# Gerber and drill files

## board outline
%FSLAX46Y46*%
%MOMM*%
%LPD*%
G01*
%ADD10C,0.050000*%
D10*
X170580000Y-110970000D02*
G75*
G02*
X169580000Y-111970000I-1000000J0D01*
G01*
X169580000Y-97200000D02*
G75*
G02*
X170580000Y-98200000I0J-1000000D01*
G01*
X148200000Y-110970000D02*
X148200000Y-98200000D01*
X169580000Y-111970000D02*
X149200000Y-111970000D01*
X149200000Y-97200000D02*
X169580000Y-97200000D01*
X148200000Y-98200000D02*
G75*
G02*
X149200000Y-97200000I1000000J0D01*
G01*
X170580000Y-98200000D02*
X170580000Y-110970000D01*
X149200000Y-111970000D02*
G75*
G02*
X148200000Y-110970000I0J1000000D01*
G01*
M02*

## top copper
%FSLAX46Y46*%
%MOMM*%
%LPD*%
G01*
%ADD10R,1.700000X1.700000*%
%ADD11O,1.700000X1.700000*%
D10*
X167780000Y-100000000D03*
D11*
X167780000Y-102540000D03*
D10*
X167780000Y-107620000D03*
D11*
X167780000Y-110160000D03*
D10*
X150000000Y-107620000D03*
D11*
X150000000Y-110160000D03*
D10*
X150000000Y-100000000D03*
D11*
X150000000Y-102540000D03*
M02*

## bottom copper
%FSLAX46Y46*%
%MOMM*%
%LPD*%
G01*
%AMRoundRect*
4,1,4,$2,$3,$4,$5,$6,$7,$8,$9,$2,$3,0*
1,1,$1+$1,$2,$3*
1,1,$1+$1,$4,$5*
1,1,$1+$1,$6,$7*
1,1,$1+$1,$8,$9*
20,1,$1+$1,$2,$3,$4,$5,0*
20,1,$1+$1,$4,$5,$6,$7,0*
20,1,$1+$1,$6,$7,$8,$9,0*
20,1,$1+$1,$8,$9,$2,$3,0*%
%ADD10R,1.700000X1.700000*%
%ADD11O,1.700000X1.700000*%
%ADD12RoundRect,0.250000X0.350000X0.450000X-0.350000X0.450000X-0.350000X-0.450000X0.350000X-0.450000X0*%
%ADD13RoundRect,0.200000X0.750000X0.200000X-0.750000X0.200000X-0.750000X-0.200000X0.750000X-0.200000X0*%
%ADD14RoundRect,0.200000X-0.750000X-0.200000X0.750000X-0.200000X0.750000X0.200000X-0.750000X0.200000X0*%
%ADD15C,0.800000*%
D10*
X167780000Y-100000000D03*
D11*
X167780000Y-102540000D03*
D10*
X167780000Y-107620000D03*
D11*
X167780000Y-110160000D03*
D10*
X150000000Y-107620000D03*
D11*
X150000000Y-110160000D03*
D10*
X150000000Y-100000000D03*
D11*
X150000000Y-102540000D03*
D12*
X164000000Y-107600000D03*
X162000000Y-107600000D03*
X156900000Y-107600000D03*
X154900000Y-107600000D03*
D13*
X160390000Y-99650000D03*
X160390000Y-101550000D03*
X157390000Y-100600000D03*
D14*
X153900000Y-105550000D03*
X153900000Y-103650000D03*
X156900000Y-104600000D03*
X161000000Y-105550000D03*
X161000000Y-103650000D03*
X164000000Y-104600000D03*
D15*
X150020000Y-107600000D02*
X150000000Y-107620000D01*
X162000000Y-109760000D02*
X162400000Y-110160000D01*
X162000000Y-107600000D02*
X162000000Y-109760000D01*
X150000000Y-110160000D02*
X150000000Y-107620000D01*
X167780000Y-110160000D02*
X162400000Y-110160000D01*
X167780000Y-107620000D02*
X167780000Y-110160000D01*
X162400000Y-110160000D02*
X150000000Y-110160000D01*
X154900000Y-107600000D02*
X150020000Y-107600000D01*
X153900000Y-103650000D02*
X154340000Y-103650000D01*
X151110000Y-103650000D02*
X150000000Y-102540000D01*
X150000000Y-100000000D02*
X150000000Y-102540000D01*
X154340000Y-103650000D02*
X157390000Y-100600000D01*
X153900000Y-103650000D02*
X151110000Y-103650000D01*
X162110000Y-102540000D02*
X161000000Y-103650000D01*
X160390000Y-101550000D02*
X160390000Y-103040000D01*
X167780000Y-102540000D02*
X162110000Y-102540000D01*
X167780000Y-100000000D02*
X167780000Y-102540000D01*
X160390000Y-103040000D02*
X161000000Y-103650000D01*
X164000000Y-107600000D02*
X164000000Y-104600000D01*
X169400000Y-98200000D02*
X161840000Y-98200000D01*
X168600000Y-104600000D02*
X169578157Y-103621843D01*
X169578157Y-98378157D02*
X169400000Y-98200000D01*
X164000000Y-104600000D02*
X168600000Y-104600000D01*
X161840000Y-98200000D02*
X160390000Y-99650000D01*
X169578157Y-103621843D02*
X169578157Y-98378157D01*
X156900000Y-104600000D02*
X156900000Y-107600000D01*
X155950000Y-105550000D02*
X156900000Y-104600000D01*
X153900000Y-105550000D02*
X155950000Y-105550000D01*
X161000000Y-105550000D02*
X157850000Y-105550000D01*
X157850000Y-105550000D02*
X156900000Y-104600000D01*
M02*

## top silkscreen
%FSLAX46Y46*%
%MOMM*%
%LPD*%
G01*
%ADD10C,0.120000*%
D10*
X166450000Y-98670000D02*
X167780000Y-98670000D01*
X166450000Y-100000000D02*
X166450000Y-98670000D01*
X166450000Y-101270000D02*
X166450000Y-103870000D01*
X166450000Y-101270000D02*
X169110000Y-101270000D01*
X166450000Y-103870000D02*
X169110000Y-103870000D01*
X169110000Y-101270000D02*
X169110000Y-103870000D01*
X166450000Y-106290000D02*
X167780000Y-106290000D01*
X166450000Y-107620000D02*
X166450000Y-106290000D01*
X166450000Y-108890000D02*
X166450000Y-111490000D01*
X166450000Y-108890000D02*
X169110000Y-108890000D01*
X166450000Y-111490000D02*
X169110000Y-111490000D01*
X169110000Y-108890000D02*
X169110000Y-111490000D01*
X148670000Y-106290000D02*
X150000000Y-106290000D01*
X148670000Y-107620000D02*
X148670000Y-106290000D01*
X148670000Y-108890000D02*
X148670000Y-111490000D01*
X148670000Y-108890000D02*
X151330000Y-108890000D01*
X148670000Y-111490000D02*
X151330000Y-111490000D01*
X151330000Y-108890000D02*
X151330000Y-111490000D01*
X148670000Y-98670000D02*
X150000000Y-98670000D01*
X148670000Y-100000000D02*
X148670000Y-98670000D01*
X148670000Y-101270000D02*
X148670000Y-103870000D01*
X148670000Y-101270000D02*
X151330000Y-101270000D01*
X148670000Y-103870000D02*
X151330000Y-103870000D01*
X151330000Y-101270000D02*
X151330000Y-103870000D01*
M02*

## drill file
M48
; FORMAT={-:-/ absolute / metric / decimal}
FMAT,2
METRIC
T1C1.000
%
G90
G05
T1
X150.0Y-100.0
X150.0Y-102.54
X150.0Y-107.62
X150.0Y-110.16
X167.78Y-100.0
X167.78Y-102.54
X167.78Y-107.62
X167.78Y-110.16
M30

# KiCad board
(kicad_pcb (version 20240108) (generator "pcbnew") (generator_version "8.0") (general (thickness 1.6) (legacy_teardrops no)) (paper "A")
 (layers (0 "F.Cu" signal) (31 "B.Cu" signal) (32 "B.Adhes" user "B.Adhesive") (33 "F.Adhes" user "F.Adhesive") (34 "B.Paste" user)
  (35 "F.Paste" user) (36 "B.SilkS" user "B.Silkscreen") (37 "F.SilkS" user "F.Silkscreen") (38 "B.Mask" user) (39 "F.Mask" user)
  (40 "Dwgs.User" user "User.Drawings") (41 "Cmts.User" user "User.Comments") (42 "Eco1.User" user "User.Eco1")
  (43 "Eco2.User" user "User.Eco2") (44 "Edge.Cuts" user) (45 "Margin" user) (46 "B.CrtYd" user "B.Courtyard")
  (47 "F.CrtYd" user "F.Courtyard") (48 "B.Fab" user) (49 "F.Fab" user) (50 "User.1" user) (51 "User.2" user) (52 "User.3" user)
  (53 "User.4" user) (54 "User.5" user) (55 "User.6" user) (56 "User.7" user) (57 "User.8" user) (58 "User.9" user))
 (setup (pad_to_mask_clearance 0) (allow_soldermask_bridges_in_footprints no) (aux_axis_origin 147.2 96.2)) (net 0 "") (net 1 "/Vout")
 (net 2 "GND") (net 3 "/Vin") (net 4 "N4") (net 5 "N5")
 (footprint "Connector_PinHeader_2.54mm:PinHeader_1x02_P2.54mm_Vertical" (layer "F.Cu") (at 167.78 100)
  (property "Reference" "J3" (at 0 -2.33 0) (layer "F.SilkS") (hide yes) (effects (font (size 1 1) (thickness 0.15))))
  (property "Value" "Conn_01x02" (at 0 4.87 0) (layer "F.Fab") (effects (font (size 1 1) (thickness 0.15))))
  (fp_line (start -1.33 -1.33) (end 0 -1.33) (stroke (width 0.12) (type solid)) (layer "F.SilkS"))
  (fp_line (start -1.33 0) (end -1.33 -1.33) (stroke (width 0.12) (type solid)) (layer "F.SilkS"))
  (fp_line (start -1.33 1.27) (end -1.33 3.87) (stroke (width 0.12) (type solid)) (layer "F.SilkS"))
  (fp_line (start -1.33 1.27) (end 1.33 1.27) (stroke (width 0.12) (type solid)) (layer "F.SilkS"))
  (fp_line (start -1.33 3.87) (end 1.33 3.87) (stroke (width 0.12) (type solid)) (layer "F.SilkS"))
  (fp_line (start 1.33 1.27) (end 1.33 3.87) (stroke (width 0.12) (type solid)) (layer "F.SilkS"))
  (pad "1" thru_hole rect (at 0 0) (size 1.7 1.7) (drill 1) (layers "*.Cu" "*.Mask") (remove_unused_layers no) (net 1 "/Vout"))
  (pad "2" thru_hole oval (at 0 2.54) (size 1.7 1.7) (drill 1) (layers "*.Cu" "*.Mask") (remove_unused_layers no) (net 1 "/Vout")))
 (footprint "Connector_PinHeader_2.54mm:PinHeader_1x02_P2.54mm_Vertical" (layer "F.Cu") (at 167.78 107.62)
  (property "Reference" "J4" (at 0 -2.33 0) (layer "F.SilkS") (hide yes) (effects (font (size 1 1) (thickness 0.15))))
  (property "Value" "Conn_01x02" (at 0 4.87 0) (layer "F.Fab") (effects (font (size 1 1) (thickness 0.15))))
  (fp_line (start -1.33 -1.33) (end 0 -1.33) (stroke (width 0.12) (type solid)) (layer "F.SilkS"))
  (fp_line (start -1.33 0) (end -1.33 -1.33) (stroke (width 0.12) (type solid)) (layer "F.SilkS"))
  (fp_line (start -1.33 1.27) (end -1.33 3.87) (stroke (width 0.12) (type solid)) (layer "F.SilkS"))
  (fp_line (start -1.33 1.27) (end 1.33 1.27) (stroke (width 0.12) (type solid)) (layer "F.SilkS"))
  (fp_line (start -1.33 3.87) (end 1.33 3.87) (stroke (width 0.12) (type solid)) (layer "F.SilkS"))
  (fp_line (start 1.33 1.27) (end 1.33 3.87) (stroke (width 0.12) (type solid)) (layer "F.SilkS"))
  (pad "1" thru_hole rect (at 0 0) (size 1.7 1.7) (drill 1) (layers "*.Cu" "*.Mask") (remove_unused_layers no) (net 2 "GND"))
  (pad "2" thru_hole oval (at 0 2.54) (size 1.7 1.7) (drill 1) (layers "*.Cu" "*.Mask") (remove_unused_layers no) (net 2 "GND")))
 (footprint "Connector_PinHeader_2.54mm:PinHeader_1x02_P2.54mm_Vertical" (layer "F.Cu") (at 150 107.62)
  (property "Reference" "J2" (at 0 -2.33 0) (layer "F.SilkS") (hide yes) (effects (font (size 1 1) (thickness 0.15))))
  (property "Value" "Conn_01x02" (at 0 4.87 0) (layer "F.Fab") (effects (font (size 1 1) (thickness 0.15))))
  (fp_line (start -1.33 -1.33) (end 0 -1.33) (stroke (width 0.12) (type solid)) (layer "F.SilkS"))
  (fp_line (start -1.33 0) (end -1.33 -1.33) (stroke (width 0.12) (type solid)) (layer "F.SilkS"))
  (fp_line (start -1.33 1.27) (end -1.33 3.87) (stroke (width 0.12) (type solid)) (layer "F.SilkS"))
  (fp_line (start -1.33 1.27) (end 1.33 1.27) (stroke (width 0.12) (type solid)) (layer "F.SilkS"))
  (fp_line (start -1.33 3.87) (end 1.33 3.87) (stroke (width 0.12) (type solid)) (layer "F.SilkS"))
  (fp_line (start 1.33 1.27) (end 1.33 3.87) (stroke (width 0.12) (type solid)) (layer "F.SilkS"))
  (pad "1" thru_hole rect (at 0 0) (size 1.7 1.7) (drill 1) (layers "*.Cu" "*.Mask") (remove_unused_layers no) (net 2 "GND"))
  (pad "2" thru_hole oval (at 0 2.54) (size 1.7 1.7) (drill 1) (layers "*.Cu" "*.Mask") (remove_unused_layers no) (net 2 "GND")))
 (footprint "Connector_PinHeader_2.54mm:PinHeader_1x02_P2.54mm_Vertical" (layer "F.Cu") (at 150 100)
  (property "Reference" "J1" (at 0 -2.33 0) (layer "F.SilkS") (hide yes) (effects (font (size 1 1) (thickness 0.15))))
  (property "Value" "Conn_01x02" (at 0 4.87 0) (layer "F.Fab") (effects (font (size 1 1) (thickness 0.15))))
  (fp_line (start -1.33 -1.33) (end 0 -1.33) (stroke (width 0.12) (type solid)) (layer "F.SilkS"))
  (fp_line (start -1.33 0) (end -1.33 -1.33) (stroke (width 0.12) (type solid)) (layer "F.SilkS"))
  (fp_line (start -1.33 1.27) (end -1.33 3.87) (stroke (width 0.12) (type solid)) (layer "F.SilkS"))
  (fp_line (start -1.33 1.27) (end 1.33 1.27) (stroke (width 0.12) (type solid)) (layer "F.SilkS"))
  (fp_line (start -1.33 3.87) (end 1.33 3.87) (stroke (width 0.12) (type solid)) (layer "F.SilkS"))
  (fp_line (start 1.33 1.27) (end 1.33 3.87) (stroke (width 0.12) (type solid)) (layer "F.SilkS"))
  (pad "1" thru_hole rect (at 0 0) (size 1.7 1.7) (drill 1) (layers "*.Cu" "*.Mask") (remove_unused_layers no) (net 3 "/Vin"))
  (pad "2" thru_hole oval (at 0 2.54) (size 1.7 1.7) (drill 1) (layers "*.Cu" "*.Mask") (remove_unused_layers no) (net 3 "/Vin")))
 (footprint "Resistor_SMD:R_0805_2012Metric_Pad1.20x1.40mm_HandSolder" (layer "B.Cu") (at 163 107.6 180)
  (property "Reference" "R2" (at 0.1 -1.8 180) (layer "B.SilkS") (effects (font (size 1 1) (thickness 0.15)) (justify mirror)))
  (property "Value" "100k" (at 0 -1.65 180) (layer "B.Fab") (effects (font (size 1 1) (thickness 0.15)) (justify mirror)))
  (pad "1" smd roundrect (at -1 0 180) (size 1.2 1.4) (layers "B.Cu" "B.Paste" "B.Mask") (roundrect_rratio 0.208333) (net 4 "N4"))
  (pad "2" smd roundrect (at 1 0 180) (size 1.2 1.4) (layers "B.Cu" "B.Paste" "B.Mask") (roundrect_rratio 0.208333) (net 2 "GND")))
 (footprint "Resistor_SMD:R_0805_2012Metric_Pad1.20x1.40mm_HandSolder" (layer "B.Cu") (at 155.9 107.6 180)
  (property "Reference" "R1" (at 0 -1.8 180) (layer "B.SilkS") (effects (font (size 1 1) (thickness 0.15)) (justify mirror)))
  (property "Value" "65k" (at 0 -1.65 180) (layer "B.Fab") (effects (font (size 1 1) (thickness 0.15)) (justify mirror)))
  (pad "1" smd roundrect (at -1 0 180) (size 1.2 1.4) (layers "B.Cu" "B.Paste" "B.Mask") (roundrect_rratio 0.208333) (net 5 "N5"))
  (pad "2" smd roundrect (at 1 0 180) (size 1.2 1.4) (layers "B.Cu" "B.Paste" "B.Mask") (roundrect_rratio 0.208333) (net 2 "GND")))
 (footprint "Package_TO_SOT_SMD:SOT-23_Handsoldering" (layer "B.Cu") (at 158.89 100.6 180)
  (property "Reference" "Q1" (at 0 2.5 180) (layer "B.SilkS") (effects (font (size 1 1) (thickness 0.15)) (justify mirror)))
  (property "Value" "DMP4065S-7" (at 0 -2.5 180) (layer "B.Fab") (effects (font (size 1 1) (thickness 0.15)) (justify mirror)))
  (pad "1" smd roundrect (at -1.5 0.95 180) (size 1.9 0.8) (layers "B.Cu" "B.Paste" "B.Mask") (roundrect_rratio 0.25) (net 4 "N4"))
  (pad "2" smd roundrect (at -1.5 -0.95 180) (size 1.9 0.8) (layers "B.Cu" "B.Paste" "B.Mask") (roundrect_rratio 0.25) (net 1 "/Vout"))
  (pad "3" smd roundrect (at 1.5 0 180) (size 1.9 0.8) (layers "B.Cu" "B.Paste" "B.Mask") (roundrect_rratio 0.25) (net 3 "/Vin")))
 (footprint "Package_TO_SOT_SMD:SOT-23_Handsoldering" (layer "B.Cu") (at 155.4 104.6)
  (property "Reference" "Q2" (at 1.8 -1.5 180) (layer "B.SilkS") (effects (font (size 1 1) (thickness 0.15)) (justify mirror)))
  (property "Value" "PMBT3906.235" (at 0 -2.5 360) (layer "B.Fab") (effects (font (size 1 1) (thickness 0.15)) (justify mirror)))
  (pad "1" smd roundrect (at -1.5 0.95) (size 1.9 0.8) (layers "B.Cu" "B.Paste" "B.Mask") (roundrect_rratio 0.25) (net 5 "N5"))
  (pad "2" smd roundrect (at -1.5 -0.95) (size 1.9 0.8) (layers "B.Cu" "B.Paste" "B.Mask") (roundrect_rratio 0.25) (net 3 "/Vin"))
  (pad "3" smd roundrect (at 1.5 0) (size 1.9 0.8) (layers "B.Cu" "B.Paste" "B.Mask") (roundrect_rratio 0.25) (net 5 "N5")))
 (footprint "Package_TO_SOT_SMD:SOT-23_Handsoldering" (layer "B.Cu") (at 162.5 104.6)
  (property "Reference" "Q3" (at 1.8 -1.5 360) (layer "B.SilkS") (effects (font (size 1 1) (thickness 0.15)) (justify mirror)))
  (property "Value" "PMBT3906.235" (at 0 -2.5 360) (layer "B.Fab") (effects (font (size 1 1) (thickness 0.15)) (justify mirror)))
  (pad "1" smd roundrect (at -1.5 0.95) (size 1.9 0.8) (layers "B.Cu" "B.Paste" "B.Mask") (roundrect_rratio 0.25) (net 5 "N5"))
  (pad "2" smd roundrect (at -1.5 -0.95) (size 1.9 0.8) (layers "B.Cu" "B.Paste" "B.Mask") (roundrect_rratio 0.25) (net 1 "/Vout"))
  (pad "3" smd roundrect (at 1.5 0) (size 1.9 0.8) (layers "B.Cu" "B.Paste" "B.Mask") (roundrect_rratio 0.25) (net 4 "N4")))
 (gr_arc (start 170.58 110.97) (mid 170.287107 111.677107) (end 169.58 111.97) (stroke (width 0.05) (type default)) (layer "Edge.Cuts"))
 (gr_arc (start 169.58 97.2) (mid 170.287107 97.492893) (end 170.58 98.2) (stroke (width 0.05) (type default)) (layer "Edge.Cuts"))
 (gr_line (start 148.2 110.97) (end 148.2 98.2) (stroke (width 0.05) (type default)) (layer "Edge.Cuts"))
 (gr_line (start 169.58 111.97) (end 149.2 111.97) (stroke (width 0.05) (type default)) (layer "Edge.Cuts"))
 (gr_line (start 149.2 97.2) (end 169.58 97.2) (stroke (width 0.05) (type default)) (layer "Edge.Cuts"))
 (gr_arc (start 148.2 98.2) (mid 148.492893 97.492893) (end 149.2 97.2) (stroke (width 0.05) (type default)) (layer "Edge.Cuts"))
 (gr_line (start 170.58 98.2) (end 170.58 110.97) (stroke (width 0.05) (type default)) (layer "Edge.Cuts"))
 (gr_arc (start 149.2 111.97) (mid 148.492893 111.677107) (end 148.2 110.97) (stroke (width 0.05) (type default)) (layer "Edge.Cuts"))
 (segment (start 150.02 107.6) (end 150 107.62) (width 0.8) (layer "B.Cu") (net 2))
 (segment (start 162 109.76) (end 162.4 110.16) (width 0.8) (layer "B.Cu") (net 2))
 (segment (start 162 107.6) (end 162 109.76) (width 0.8) (layer "B.Cu") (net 2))
 (segment (start 150 110.16) (end 150 107.62) (width 0.8) (layer "B.Cu") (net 2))
 (segment (start 167.78 110.16) (end 162.4 110.16) (width 0.8) (layer "B.Cu") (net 2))
 (segment (start 167.78 107.62) (end 167.78 110.16) (width 0.8) (layer "B.Cu") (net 2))
 (segment (start 162.4 110.16) (end 150 110.16) (width 0.8) (layer "B.Cu") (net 2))
 (segment (start 154.9 107.6) (end 150.02 107.6) (width 0.8) (layer "B.Cu") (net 2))
 (segment (start 153.9 103.65) (end 154.34 103.65) (width 0.8) (layer "B.Cu") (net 3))
 (segment (start 151.11 103.65) (end 150 102.54) (width 0.8) (layer "B.Cu") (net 3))
 (segment (start 150 100) (end 150 102.54) (width 0.8) (layer "B.Cu") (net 3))
 (segment (start 154.34 103.65) (end 157.39 100.6) (width 0.8) (layer "B.Cu") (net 3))
 (segment (start 153.9 103.65) (end 151.11 103.65) (width 0.8) (layer "B.Cu") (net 3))
 (segment (start 162.11 102.54) (end 161 103.65) (width 0.8) (layer "B.Cu") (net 1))
 (segment (start 160.39 101.55) (end 160.39 103.04) (width 0.8) (layer "B.Cu") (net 1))
 (segment (start 167.78 102.54) (end 162.11 102.54) (width 0.8) (layer "B.Cu") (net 1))
 (segment (start 167.78 100) (end 167.78 102.54) (width 0.8) (layer "B.Cu") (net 1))
 (segment (start 160.39 103.04) (end 161 103.65) (width 0.8) (layer "B.Cu") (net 1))
 (segment (start 164 107.6) (end 164 104.6) (width 0.8) (layer "B.Cu") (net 4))
 (segment (start 169.4 98.2) (end 161.84 98.2) (width 0.8) (layer "B.Cu") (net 4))
 (segment (start 168.6 104.6) (end 169.578157 103.621843) (width 0.8) (layer "B.Cu") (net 4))
 (segment (start 169.578157 98.378157) (end 169.4 98.2) (width 0.8) (layer "B.Cu") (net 4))
 (segment (start 164 104.6) (end 168.6 104.6) (width 0.8) (layer "B.Cu") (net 4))
 (segment (start 161.84 98.2) (end 160.39 99.65) (width 0.8) (layer "B.Cu") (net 4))
 (segment (start 169.578157 103.621843) (end 169.578157 98.378157) (width 0.8) (layer "B.Cu") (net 4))
 (segment (start 156.9 104.6) (end 156.9 107.6) (width 0.8) (layer "B.Cu") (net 5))
 (segment (start 155.95 105.55) (end 156.9 104.6) (width 0.8) (layer "B.Cu") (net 5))
 (segment (start 153.9 105.55) (end 155.95 105.55) (width 0.8) (layer "B.Cu") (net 5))
 (segment (start 161 105.55) (end 157.85 105.55) (width 0.8) (layer "B.Cu") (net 5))
 (segment (start 157.85 105.55) (end 156.9 104.6) (width 0.8) (layer "B.Cu") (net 5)))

